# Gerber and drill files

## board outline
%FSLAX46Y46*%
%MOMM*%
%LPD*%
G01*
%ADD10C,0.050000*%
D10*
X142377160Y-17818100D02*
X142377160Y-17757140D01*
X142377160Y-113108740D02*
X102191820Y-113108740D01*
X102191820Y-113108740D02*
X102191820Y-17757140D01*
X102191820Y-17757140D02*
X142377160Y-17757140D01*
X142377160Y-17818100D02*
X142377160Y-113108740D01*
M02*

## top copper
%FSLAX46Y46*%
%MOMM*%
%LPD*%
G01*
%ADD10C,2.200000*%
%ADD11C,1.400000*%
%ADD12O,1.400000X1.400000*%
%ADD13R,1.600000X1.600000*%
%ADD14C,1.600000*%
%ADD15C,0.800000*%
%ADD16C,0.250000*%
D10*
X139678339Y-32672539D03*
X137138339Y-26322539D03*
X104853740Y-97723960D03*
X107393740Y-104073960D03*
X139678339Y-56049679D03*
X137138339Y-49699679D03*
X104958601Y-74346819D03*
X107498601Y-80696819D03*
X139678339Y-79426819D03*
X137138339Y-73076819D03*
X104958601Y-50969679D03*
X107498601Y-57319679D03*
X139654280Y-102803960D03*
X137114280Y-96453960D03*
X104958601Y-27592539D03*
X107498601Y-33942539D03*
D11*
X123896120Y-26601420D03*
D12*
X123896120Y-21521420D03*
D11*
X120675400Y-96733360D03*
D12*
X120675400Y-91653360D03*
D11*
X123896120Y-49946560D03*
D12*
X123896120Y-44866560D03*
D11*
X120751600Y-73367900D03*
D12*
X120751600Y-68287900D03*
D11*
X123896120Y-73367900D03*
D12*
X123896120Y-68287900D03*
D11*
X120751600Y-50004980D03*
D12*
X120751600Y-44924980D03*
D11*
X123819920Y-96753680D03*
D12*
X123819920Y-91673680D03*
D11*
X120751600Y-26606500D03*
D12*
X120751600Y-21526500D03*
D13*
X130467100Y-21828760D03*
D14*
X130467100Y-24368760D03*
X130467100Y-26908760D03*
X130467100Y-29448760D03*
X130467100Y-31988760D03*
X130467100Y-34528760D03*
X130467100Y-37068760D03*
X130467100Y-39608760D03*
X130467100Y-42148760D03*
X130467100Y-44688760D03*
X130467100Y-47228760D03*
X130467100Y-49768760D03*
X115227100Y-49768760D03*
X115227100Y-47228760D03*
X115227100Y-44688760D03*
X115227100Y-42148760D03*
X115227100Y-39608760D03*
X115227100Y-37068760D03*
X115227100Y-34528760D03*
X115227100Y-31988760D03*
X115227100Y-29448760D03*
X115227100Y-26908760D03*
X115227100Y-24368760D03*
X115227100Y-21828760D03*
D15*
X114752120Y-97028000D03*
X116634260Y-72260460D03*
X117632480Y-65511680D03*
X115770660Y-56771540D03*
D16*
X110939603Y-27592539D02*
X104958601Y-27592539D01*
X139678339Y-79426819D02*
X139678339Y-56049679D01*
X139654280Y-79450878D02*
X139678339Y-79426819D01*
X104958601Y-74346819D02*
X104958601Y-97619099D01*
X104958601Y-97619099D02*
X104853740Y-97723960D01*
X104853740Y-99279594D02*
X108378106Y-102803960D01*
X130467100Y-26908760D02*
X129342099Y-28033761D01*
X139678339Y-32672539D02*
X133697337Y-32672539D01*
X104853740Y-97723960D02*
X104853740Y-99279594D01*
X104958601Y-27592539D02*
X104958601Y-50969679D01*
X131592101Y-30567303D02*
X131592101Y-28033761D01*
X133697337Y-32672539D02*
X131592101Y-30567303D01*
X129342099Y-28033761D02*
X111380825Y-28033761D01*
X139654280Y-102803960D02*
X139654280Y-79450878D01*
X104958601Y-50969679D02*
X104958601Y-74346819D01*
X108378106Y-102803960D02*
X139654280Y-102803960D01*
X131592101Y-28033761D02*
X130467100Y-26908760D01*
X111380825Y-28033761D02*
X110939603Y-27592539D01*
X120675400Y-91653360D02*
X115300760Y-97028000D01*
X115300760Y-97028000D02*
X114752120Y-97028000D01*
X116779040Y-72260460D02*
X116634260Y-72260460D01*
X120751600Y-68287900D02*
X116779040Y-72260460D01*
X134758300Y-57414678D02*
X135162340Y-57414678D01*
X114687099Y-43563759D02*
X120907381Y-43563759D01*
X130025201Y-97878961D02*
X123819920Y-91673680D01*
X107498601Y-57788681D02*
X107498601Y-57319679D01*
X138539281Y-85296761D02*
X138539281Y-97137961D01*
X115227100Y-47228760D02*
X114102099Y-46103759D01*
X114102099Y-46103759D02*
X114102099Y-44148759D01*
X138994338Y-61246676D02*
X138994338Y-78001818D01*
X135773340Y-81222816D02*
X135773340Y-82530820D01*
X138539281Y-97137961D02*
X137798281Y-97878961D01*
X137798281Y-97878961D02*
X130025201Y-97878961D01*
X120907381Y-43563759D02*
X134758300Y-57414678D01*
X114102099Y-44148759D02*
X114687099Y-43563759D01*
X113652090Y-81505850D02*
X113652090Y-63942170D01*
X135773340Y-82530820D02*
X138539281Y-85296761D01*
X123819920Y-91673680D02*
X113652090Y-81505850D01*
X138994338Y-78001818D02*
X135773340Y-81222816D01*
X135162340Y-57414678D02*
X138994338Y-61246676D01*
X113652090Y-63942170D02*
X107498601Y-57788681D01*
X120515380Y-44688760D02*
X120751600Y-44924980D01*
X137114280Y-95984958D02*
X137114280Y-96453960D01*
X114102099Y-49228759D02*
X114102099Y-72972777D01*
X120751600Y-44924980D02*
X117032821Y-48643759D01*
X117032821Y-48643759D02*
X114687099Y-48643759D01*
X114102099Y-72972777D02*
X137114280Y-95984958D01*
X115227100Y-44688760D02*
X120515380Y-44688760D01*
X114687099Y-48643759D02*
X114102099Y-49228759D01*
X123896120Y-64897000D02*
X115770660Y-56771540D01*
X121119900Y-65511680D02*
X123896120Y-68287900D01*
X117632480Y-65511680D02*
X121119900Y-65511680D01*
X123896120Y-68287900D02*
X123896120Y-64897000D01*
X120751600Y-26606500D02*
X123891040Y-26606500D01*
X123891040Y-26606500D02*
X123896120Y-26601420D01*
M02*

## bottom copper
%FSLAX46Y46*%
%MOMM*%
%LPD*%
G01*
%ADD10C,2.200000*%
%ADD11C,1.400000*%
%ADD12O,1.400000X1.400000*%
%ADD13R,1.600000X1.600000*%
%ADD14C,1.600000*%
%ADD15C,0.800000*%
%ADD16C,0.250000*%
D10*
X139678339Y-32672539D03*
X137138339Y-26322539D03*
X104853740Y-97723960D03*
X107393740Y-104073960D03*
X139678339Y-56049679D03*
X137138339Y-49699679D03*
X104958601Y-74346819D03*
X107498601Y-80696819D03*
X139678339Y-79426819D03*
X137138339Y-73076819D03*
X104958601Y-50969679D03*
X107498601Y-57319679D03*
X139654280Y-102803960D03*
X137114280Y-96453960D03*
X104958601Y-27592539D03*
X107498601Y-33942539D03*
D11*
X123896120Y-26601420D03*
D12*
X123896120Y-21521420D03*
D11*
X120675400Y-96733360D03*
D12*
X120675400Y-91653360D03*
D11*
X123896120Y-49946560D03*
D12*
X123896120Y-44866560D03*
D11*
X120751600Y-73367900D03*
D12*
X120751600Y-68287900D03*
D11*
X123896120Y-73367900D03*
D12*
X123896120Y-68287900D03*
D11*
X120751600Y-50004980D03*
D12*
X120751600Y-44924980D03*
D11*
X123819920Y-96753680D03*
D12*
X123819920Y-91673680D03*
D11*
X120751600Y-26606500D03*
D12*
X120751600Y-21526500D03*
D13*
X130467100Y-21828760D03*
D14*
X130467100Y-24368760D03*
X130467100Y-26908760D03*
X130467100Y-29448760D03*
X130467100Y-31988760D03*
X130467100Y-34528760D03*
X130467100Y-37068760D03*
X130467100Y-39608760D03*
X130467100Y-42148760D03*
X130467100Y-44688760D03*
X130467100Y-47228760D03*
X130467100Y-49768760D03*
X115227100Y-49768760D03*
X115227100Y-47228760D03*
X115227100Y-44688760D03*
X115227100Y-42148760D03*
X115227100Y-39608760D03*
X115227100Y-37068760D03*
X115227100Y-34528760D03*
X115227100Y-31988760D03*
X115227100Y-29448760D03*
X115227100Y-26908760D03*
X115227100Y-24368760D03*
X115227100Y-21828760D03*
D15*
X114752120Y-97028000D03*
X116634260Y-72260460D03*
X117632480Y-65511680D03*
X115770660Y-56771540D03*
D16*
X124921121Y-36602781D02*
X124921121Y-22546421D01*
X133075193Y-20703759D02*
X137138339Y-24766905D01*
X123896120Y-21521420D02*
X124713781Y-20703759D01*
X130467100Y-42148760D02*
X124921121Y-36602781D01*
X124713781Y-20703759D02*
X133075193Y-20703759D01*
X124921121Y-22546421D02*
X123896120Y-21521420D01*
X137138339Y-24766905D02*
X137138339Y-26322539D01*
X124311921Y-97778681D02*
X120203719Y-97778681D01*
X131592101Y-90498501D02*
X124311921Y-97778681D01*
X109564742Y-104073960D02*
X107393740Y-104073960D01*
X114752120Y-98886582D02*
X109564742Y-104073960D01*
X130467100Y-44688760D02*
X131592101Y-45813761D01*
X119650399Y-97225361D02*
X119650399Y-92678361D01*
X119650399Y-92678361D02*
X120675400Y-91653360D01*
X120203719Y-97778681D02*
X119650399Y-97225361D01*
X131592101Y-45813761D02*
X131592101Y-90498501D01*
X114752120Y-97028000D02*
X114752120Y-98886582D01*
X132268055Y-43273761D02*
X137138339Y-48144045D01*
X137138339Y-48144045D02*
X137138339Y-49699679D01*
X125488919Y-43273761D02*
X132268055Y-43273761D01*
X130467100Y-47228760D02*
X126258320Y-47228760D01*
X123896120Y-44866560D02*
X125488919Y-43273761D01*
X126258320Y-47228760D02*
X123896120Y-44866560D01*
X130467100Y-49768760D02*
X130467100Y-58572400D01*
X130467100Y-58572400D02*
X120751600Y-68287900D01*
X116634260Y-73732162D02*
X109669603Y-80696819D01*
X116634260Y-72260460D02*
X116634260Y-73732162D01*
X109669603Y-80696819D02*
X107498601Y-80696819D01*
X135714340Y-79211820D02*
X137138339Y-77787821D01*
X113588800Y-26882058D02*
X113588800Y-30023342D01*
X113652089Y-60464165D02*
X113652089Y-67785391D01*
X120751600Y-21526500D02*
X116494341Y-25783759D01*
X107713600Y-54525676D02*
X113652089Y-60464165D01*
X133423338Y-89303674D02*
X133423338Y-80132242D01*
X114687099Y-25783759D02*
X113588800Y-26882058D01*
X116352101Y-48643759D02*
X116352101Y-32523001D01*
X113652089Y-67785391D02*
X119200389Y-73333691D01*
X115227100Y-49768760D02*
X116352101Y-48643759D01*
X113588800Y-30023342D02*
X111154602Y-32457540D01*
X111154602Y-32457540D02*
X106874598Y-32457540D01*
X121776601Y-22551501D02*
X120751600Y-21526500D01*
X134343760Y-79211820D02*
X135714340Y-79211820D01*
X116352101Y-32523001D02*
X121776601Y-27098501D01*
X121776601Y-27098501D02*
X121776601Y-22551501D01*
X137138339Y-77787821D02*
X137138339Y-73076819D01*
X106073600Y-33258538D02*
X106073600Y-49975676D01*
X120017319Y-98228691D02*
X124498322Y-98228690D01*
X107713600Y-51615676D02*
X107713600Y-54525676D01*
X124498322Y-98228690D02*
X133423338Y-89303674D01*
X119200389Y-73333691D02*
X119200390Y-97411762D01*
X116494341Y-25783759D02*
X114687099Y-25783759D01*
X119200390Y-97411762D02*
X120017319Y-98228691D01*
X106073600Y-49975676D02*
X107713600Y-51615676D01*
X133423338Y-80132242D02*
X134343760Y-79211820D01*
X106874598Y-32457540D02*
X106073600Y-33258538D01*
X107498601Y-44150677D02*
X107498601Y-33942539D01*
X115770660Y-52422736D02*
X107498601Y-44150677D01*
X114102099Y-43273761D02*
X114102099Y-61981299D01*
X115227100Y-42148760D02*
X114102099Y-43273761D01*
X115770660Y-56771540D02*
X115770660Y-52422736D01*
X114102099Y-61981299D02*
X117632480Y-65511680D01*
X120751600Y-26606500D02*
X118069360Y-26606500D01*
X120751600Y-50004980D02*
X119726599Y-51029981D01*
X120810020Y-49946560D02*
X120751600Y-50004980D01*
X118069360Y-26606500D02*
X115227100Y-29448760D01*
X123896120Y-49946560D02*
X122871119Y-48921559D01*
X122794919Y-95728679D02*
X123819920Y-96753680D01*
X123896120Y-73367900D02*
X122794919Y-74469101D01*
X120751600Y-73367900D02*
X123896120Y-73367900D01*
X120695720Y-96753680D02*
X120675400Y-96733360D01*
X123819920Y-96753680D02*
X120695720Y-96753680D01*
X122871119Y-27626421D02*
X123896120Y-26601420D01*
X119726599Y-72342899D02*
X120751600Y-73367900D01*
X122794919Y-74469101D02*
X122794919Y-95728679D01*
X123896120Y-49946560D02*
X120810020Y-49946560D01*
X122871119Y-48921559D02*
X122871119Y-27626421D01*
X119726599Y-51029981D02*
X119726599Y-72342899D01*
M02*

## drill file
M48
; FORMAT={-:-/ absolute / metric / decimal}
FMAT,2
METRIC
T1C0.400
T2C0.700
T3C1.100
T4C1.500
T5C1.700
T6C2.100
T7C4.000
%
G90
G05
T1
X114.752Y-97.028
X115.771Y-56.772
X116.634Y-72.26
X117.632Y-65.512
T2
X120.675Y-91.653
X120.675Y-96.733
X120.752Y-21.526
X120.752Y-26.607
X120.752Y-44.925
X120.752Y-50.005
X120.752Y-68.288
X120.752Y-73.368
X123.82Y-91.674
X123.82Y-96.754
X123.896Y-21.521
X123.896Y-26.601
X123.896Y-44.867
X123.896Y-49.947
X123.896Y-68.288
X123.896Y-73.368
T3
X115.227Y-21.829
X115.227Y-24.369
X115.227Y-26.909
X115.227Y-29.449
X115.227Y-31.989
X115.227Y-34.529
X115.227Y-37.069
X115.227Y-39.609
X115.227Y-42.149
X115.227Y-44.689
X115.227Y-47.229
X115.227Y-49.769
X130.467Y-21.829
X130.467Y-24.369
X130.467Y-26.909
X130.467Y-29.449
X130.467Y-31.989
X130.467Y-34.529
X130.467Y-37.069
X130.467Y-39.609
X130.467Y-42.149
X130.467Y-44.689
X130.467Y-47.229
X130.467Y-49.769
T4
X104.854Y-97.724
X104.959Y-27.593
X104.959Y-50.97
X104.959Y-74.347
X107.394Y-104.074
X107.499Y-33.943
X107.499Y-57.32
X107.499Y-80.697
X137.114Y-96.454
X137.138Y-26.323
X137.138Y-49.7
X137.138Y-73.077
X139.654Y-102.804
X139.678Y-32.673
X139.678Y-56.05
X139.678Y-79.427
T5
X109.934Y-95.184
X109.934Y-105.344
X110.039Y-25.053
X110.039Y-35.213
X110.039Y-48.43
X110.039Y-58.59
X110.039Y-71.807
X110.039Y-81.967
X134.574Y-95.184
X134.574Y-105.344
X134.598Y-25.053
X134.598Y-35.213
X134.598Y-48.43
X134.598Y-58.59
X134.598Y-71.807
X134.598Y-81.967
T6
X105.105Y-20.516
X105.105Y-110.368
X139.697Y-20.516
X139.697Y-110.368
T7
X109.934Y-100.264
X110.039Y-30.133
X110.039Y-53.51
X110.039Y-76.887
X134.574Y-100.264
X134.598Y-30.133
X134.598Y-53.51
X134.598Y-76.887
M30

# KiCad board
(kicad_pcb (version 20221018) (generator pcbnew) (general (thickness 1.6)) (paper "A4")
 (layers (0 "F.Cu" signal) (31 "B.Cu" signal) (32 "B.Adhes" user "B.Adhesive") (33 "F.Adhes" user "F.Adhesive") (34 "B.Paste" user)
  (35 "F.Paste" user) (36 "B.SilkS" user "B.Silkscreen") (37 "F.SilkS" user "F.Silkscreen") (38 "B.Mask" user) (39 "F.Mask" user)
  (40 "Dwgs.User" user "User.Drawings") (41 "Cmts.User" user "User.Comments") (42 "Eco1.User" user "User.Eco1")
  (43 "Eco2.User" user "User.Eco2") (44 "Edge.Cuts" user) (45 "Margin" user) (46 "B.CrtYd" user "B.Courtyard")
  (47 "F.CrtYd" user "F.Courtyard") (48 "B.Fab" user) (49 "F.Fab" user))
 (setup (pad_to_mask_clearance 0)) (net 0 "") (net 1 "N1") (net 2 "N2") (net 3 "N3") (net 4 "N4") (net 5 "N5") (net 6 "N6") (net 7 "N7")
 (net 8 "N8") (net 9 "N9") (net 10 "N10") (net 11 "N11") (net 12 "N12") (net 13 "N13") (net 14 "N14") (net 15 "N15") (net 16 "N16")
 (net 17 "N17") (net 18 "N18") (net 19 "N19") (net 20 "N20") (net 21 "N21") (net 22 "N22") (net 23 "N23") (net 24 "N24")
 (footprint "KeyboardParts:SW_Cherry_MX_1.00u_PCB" (layer "F.Cu") (at 139.678339 32.672539 -90)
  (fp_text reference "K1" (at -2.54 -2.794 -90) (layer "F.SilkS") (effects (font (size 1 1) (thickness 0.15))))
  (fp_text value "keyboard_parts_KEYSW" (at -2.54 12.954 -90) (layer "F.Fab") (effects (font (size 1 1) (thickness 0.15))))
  (pad "" np_thru_hole circle (at -7.62 5.08 270) (size 1.7 1.7) (drill 1.7) (layers "*.Cu" "*.Mask"))
  (pad "" np_thru_hole circle (at -2.54 5.08 270) (size 4 4) (drill 4) (layers "*.Cu" "*.Mask"))
  (pad "" np_thru_hole circle (at 2.54 5.08 270) (size 1.7 1.7) (drill 1.7) (layers "*.Cu" "*.Mask"))
  (pad "1" thru_hole circle (at 0 0 270) (size 2.2 2.2) (drill 1.5) (layers "*.Cu" "*.Mask") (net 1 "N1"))
  (pad "2" thru_hole circle (at -6.35 2.54 270) (size 2.2 2.2) (drill 1.5) (layers "*.Cu" "*.Mask") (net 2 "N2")))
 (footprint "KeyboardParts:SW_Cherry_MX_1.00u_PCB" (layer "F.Cu") (at 104.85374 97.72396 90)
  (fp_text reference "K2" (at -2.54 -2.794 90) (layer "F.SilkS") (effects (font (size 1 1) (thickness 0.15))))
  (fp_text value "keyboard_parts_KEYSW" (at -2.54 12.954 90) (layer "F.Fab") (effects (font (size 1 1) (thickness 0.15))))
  (pad "" np_thru_hole circle (at -7.62 5.08 90) (size 1.7 1.7) (drill 1.7) (layers "*.Cu" "*.Mask"))
  (pad "" np_thru_hole circle (at -2.54 5.08 90) (size 4 4) (drill 4) (layers "*.Cu" "*.Mask"))
  (pad "" np_thru_hole circle (at 2.54 5.08 90) (size 1.7 1.7) (drill 1.7) (layers "*.Cu" "*.Mask"))
  (pad "1" thru_hole circle (at 0 0 90) (size 2.2 2.2) (drill 1.5) (layers "*.Cu" "*.Mask") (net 1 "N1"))
  (pad "2" thru_hole circle (at -6.35 2.54 90) (size 2.2 2.2) (drill 1.5) (layers "*.Cu" "*.Mask") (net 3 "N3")))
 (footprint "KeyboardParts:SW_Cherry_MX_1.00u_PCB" (layer "F.Cu") (at 139.678339 56.049679 -90)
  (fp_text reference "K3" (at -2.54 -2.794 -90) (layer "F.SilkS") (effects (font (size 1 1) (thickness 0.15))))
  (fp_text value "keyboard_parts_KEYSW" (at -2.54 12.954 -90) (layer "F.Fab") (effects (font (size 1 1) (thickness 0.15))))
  (pad "" np_thru_hole circle (at -7.62 5.08 270) (size 1.7 1.7) (drill 1.7) (layers "*.Cu" "*.Mask"))
  (pad "" np_thru_hole circle (at -2.54 5.08 270) (size 4 4) (drill 4) (layers "*.Cu" "*.Mask"))
  (pad "" np_thru_hole circle (at 2.54 5.08 270) (size 1.7 1.7) (drill 1.7) (layers "*.Cu" "*.Mask"))
  (pad "1" thru_hole circle (at 0 0 270) (size 2.2 2.2) (drill 1.5) (layers "*.Cu" "*.Mask") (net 1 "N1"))
  (pad "2" thru_hole circle (at -6.35 2.54 270) (size 2.2 2.2) (drill 1.5) (layers "*.Cu" "*.Mask") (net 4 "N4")))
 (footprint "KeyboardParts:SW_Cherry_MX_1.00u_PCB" (layer "F.Cu") (at 104.958601 74.346819 90)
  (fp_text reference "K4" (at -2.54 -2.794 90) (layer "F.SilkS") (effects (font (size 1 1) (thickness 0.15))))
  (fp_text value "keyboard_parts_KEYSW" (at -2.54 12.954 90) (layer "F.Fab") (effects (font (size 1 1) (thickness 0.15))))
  (pad "" np_thru_hole circle (at -7.62 5.08 90) (size 1.7 1.7) (drill 1.7) (layers "*.Cu" "*.Mask"))
  (pad "" np_thru_hole circle (at -2.54 5.08 90) (size 4 4) (drill 4) (layers "*.Cu" "*.Mask"))
  (pad "" np_thru_hole circle (at 2.54 5.08 90) (size 1.7 1.7) (drill 1.7) (layers "*.Cu" "*.Mask"))
  (pad "1" thru_hole circle (at 0 0 90) (size 2.2 2.2) (drill 1.5) (layers "*.Cu" "*.Mask") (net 1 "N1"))
  (pad "2" thru_hole circle (at -6.35 2.54 90) (size 2.2 2.2) (drill 1.5) (layers "*.Cu" "*.Mask") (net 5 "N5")))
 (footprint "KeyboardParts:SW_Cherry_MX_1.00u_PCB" (layer "F.Cu") (at 139.678339 79.426819 -90)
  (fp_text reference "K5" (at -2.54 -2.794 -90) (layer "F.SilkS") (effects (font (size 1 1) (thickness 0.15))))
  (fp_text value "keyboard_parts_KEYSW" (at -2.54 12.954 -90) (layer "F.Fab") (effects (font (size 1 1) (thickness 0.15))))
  (pad "" np_thru_hole circle (at -7.62 5.08 270) (size 1.7 1.7) (drill 1.7) (layers "*.Cu" "*.Mask"))
  (pad "" np_thru_hole circle (at -2.54 5.08 270) (size 4 4) (drill 4) (layers "*.Cu" "*.Mask"))
  (pad "" np_thru_hole circle (at 2.54 5.08 270) (size 1.7 1.7) (drill 1.7) (layers "*.Cu" "*.Mask"))
  (pad "1" thru_hole circle (at 0 0 270) (size 2.2 2.2) (drill 1.5) (layers "*.Cu" "*.Mask") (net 1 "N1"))
  (pad "2" thru_hole circle (at -6.35 2.54 270) (size 2.2 2.2) (drill 1.5) (layers "*.Cu" "*.Mask") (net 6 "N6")))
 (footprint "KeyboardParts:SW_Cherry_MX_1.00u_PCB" (layer "F.Cu") (at 104.958601 50.969679 90)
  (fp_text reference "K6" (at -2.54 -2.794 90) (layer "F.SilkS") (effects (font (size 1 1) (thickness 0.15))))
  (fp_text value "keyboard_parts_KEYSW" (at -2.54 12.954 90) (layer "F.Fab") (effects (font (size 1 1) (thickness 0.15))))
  (pad "" np_thru_hole circle (at -7.62 5.08 90) (size 1.7 1.7) (drill 1.7) (layers "*.Cu" "*.Mask"))
  (pad "" np_thru_hole circle (at -2.54 5.08 90) (size 4 4) (drill 4) (layers "*.Cu" "*.Mask"))
  (pad "" np_thru_hole circle (at 2.54 5.08 90) (size 1.7 1.7) (drill 1.7) (layers "*.Cu" "*.Mask"))
  (pad "1" thru_hole circle (at 0 0 90) (size 2.2 2.2) (drill 1.5) (layers "*.Cu" "*.Mask") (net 1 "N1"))
  (pad "2" thru_hole circle (at -6.35 2.54 90) (size 2.2 2.2) (drill 1.5) (layers "*.Cu" "*.Mask") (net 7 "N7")))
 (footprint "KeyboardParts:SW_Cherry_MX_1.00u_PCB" (layer "F.Cu") (at 139.65428 102.80396 -90)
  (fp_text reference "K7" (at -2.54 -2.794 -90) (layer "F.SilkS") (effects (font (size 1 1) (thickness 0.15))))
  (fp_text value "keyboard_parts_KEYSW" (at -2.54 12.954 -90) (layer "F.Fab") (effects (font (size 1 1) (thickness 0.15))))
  (pad "" np_thru_hole circle (at -7.62 5.08 270) (size 1.7 1.7) (drill 1.7) (layers "*.Cu" "*.Mask"))
  (pad "" np_thru_hole circle (at -2.54 5.08 270) (size 4 4) (drill 4) (layers "*.Cu" "*.Mask"))
  (pad "" np_thru_hole circle (at 2.54 5.08 270) (size 1.7 1.7) (drill 1.7) (layers "*.Cu" "*.Mask"))
  (pad "1" thru_hole circle (at 0 0 270) (size 2.2 2.2) (drill 1.5) (layers "*.Cu" "*.Mask") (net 1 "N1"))
  (pad "2" thru_hole circle (at -6.35 2.54 270) (size 2.2 2.2) (drill 1.5) (layers "*.Cu" "*.Mask") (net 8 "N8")))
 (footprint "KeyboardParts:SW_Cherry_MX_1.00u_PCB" (layer "F.Cu") (at 104.958601 27.592539 90)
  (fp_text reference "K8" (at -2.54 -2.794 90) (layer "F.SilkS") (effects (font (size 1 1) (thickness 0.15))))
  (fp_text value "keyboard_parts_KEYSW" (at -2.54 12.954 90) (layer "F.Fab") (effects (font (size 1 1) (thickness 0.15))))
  (pad "" np_thru_hole circle (at -7.62 5.08 90) (size 1.7 1.7) (drill 1.7) (layers "*.Cu" "*.Mask"))
  (pad "" np_thru_hole circle (at -2.54 5.08 90) (size 4 4) (drill 4) (layers "*.Cu" "*.Mask"))
  (pad "" np_thru_hole circle (at 2.54 5.08 90) (size 1.7 1.7) (drill 1.7) (layers "*.Cu" "*.Mask"))
  (pad "1" thru_hole circle (at 0 0 90) (size 2.2 2.2) (drill 1.5) (layers "*.Cu" "*.Mask") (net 1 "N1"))
  (pad "2" thru_hole circle (at -6.35 2.54 90) (size 2.2 2.2) (drill 1.5) (layers "*.Cu" "*.Mask") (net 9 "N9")))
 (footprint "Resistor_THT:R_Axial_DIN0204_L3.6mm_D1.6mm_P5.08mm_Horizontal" (layer "F.Cu") (at 123.89612 26.60142 90)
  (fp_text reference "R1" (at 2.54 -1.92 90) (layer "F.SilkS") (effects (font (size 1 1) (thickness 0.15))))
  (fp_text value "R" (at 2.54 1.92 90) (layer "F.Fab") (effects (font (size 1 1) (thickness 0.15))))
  (pad "1" thru_hole circle (at 0 0 90) (size 1.4 1.4) (drill 0.7) (layers "*.Cu" "*.Mask") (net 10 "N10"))
  (pad "2" thru_hole oval (at 5.08 0 90) (size 1.4 1.4) (drill 0.7) (layers "*.Cu" "*.Mask") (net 2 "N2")))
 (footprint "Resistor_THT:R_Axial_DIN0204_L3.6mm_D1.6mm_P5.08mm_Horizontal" (layer "F.Cu") (at 120.6754 96.73336 90)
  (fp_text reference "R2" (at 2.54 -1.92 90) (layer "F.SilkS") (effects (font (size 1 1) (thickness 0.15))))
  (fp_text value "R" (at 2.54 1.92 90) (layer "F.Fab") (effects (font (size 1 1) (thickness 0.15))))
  (pad "1" thru_hole circle (at 0 0 90) (size 1.4 1.4) (drill 0.7) (layers "*.Cu" "*.Mask") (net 10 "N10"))
  (pad "2" thru_hole oval (at 5.08 0 90) (size 1.4 1.4) (drill 0.7) (layers "*.Cu" "*.Mask") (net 3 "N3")))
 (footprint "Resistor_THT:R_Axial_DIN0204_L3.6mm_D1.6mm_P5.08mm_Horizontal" (layer "F.Cu") (at 123.89612 49.94656 90)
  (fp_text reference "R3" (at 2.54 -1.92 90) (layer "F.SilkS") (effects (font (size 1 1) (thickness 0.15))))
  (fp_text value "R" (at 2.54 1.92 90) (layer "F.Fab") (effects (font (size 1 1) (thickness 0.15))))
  (pad "1" thru_hole circle (at 0 0 90) (size 1.4 1.4) (drill 0.7) (layers "*.Cu" "*.Mask") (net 10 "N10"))
  (pad "2" thru_hole oval (at 5.08 0 90) (size 1.4 1.4) (drill 0.7) (layers "*.Cu" "*.Mask") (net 4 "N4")))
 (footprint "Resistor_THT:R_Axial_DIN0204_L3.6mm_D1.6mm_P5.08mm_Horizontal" (layer "F.Cu") (at 120.7516 73.3679 90)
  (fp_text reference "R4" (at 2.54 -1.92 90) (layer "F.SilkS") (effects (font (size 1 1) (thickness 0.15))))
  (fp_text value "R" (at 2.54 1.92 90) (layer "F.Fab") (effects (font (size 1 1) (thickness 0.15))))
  (pad "1" thru_hole circle (at 0 0 90) (size 1.4 1.4) (drill 0.7) (layers "*.Cu" "*.Mask") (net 10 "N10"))
  (pad "2" thru_hole oval (at 5.08 0 90) (size 1.4 1.4) (drill 0.7) (layers "*.Cu" "*.Mask") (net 5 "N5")))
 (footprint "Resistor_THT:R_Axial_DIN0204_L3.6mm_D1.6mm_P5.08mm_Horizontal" (layer "F.Cu") (at 123.89612 73.3679 90)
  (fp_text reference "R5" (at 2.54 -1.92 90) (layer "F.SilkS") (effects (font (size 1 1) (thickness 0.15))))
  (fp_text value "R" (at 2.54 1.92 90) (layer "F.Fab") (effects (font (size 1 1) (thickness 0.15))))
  (pad "1" thru_hole circle (at 0 0 90) (size 1.4 1.4) (drill 0.7) (layers "*.Cu" "*.Mask") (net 10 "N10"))
  (pad "2" thru_hole oval (at 5.08 0 90) (size 1.4 1.4) (drill 0.7) (layers "*.Cu" "*.Mask") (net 9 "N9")))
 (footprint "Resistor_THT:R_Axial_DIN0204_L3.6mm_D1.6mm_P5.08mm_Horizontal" (layer "F.Cu") (at 120.7516 50.00498 90)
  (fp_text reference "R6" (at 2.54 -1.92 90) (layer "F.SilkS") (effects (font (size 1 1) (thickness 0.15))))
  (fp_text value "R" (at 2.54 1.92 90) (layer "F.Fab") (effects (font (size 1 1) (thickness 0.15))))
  (pad "1" thru_hole circle (at 0 0 90) (size 1.4 1.4) (drill 0.7) (layers "*.Cu" "*.Mask") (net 10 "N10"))
  (pad "2" thru_hole oval (at 5.08 0 90) (size 1.4 1.4) (drill 0.7) (layers "*.Cu" "*.Mask") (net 8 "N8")))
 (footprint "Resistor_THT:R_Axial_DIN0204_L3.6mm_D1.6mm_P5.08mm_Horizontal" (layer "F.Cu") (at 123.81992 96.75368 90)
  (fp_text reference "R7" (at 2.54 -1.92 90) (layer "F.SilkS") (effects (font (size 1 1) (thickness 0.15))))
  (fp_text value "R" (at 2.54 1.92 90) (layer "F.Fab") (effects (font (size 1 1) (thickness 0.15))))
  (pad "1" thru_hole circle (at 0 0 90) (size 1.4 1.4) (drill 0.7) (layers "*.Cu" "*.Mask") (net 10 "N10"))
  (pad "2" thru_hole oval (at 5.08 0 90) (size 1.4 1.4) (drill 0.7) (layers "*.Cu" "*.Mask") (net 7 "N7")))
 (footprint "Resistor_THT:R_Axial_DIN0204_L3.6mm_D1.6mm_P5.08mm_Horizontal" (layer "F.Cu") (at 120.7516 26.6065 90)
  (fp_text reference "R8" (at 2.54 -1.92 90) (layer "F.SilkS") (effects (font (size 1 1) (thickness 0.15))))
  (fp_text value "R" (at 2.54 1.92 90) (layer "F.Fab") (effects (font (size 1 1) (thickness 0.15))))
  (pad "1" thru_hole circle (at 0 0 90) (size 1.4 1.4) (drill 0.7) (layers "*.Cu" "*.Mask") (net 10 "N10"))
  (pad "2" thru_hole oval (at 5.08 0 90) (size 1.4 1.4) (drill 0.7) (layers "*.Cu" "*.Mask") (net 6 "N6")))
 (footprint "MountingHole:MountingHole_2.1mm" (layer "F.Cu") (at 139.69746 110.36808)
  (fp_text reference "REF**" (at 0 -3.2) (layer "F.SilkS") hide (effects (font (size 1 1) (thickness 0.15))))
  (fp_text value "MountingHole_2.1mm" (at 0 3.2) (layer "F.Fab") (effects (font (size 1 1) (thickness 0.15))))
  (pad "" np_thru_hole circle (at 0 0) (size 2.1 2.1) (drill 2.1) (layers "*.Cu" "*.Mask")))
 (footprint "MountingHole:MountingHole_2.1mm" (layer "F.Cu") (at 105.1052 110.36808)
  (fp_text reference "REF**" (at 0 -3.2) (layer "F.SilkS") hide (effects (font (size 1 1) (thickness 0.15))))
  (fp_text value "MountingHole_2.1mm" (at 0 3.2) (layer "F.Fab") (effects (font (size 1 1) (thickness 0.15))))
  (pad "" np_thru_hole circle (at 0 0) (size 2.1 2.1) (drill 2.1) (layers "*.Cu" "*.Mask")))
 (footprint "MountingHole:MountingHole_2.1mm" (layer "F.Cu") (at 105.1052 20.51558)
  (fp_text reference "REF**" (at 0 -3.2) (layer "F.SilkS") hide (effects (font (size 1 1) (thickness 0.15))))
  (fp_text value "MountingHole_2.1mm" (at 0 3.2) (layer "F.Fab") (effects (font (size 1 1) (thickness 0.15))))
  (pad "" np_thru_hole circle (at 0 0) (size 2.1 2.1) (drill 2.1) (layers "*.Cu" "*.Mask")))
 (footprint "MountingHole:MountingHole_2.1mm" (layer "F.Cu") (at 139.69746 20.51558)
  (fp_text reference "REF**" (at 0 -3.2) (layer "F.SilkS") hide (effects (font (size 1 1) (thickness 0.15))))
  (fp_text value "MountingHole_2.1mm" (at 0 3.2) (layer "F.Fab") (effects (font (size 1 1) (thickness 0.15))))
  (pad "" np_thru_hole circle (at 0 0) (size 2.1 2.1) (drill 2.1) (layers "*.Cu" "*.Mask")))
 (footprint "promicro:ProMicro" (layer "B.Cu") (at 122.8471 35.79876 -90)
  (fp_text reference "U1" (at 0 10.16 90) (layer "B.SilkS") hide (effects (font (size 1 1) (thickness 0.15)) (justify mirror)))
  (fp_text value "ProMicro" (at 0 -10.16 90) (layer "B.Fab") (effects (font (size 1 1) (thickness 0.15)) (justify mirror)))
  (pad "1" thru_hole rect (at -13.97 -7.62 270) (size 1.6 1.6) (drill 1.1) (layers "*.Cu" "*.Mask" "B.SilkS") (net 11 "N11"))
  (pad "2" thru_hole circle (at -11.43 -7.62 270) (size 1.6 1.6) (drill 1.1) (layers "*.Cu" "*.Mask" "B.SilkS") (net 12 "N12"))
  (pad "3" thru_hole circle (at -8.89 -7.62 270) (size 1.6 1.6) (drill 1.1) (layers "*.Cu" "*.Mask" "B.SilkS") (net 1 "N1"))
  (pad "4" thru_hole circle (at -6.35 -7.62 270) (size 1.6 1.6) (drill 1.1) (layers "*.Cu" "*.Mask" "B.SilkS") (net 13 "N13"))
  (pad "5" thru_hole circle (at -3.81 -7.62 270) (size 1.6 1.6) (drill 1.1) (layers "*.Cu" "*.Mask" "B.SilkS") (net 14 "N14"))
  (pad "6" thru_hole circle (at -1.27 -7.62 270) (size 1.6 1.6) (drill 1.1) (layers "*.Cu" "*.Mask" "B.SilkS") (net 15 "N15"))
  (pad "7" thru_hole circle (at 1.27 -7.62 270) (size 1.6 1.6) (drill 1.1) (layers "*.Cu" "*.Mask" "B.SilkS") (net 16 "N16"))
  (pad "8" thru_hole circle (at 3.81 -7.62 270) (size 1.6 1.6) (drill 1.1) (layers "*.Cu" "*.Mask" "B.SilkS") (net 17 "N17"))
  (pad "9" thru_hole circle (at 6.35 -7.62 270) (size 1.6 1.6) (drill 1.1) (layers "*.Cu" "*.Mask" "B.SilkS") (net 2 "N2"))
  (pad "10" thru_hole circle (at 8.89 -7.62 270) (size 1.6 1.6) (drill 1.1) (layers "*.Cu" "*.Mask" "B.SilkS") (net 3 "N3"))
  (pad "11" thru_hole circle (at 11.43 -7.62 270) (size 1.6 1.6) (drill 1.1) (layers "*.Cu" "*.Mask" "B.SilkS") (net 4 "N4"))
  (pad "12" thru_hole circle (at 13.97 -7.62 270) (size 1.6 1.6) (drill 1.1) (layers "*.Cu" "*.Mask" "B.SilkS") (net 5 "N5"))
  (pad "13" thru_hole circle (at 13.97 7.62 270) (size 1.6 1.6) (drill 1.1) (layers "*.Cu" "*.Mask" "B.SilkS") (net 6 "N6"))
  (pad "14" thru_hole circle (at 11.43 7.62 270) (size 1.6 1.6) (drill 1.1) (layers "*.Cu" "*.Mask" "B.SilkS") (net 7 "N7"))
  (pad "15" thru_hole circle (at 8.89 7.62 270) (size 1.6 1.6) (drill 1.1) (layers "*.Cu" "*.Mask" "B.SilkS") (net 8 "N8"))
  (pad "16" thru_hole circle (at 6.35 7.62 270) (size 1.6 1.6) (drill 1.1) (layers "*.Cu" "*.Mask" "B.SilkS") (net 9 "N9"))
  (pad "17" thru_hole circle (at 3.81 7.62 270) (size 1.6 1.6) (drill 1.1) (layers "*.Cu" "*.Mask" "B.SilkS") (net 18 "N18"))
  (pad "18" thru_hole circle (at 1.27 7.62 270) (size 1.6 1.6) (drill 1.1) (layers "*.Cu" "*.Mask" "B.SilkS") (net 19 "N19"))
  (pad "19" thru_hole circle (at -1.27 7.62 270) (size 1.6 1.6) (drill 1.1) (layers "*.Cu" "*.Mask" "B.SilkS") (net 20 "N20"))
  (pad "20" thru_hole circle (at -3.81 7.62 270) (size 1.6 1.6) (drill 1.1) (layers "*.Cu" "*.Mask" "B.SilkS") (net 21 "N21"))
  (pad "21" thru_hole circle (at -6.35 7.62 270) (size 1.6 1.6) (drill 1.1) (layers "*.Cu" "*.Mask" "B.SilkS") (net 10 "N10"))
  (pad "22" thru_hole circle (at -8.89 7.62 270) (size 1.6 1.6) (drill 1.1) (layers "*.Cu" "*.Mask" "B.SilkS") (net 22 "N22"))
  (pad "23" thru_hole circle (at -11.43 7.62 270) (size 1.6 1.6) (drill 1.1) (layers "*.Cu" "*.Mask" "B.SilkS") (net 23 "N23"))
  (pad "24" thru_hole circle (at -13.97 7.62 270) (size 1.6 1.6) (drill 1.1) (layers "*.Cu" "*.Mask" "B.SilkS") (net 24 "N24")))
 (gr_line (start 142.37716 17.8181) (end 142.37716 17.75714) (stroke (width 0.05) (type solid)) (layer "Edge.Cuts"))
 (gr_line (start 142.37716 113.10874) (end 102.19182 113.10874) (stroke (width 0.05) (type solid)) (layer "Edge.Cuts"))
 (gr_line (start 102.19182 113.10874) (end 102.19182 17.75714) (stroke (width 0.05) (type solid)) (layer "Edge.Cuts"))
 (gr_line (start 102.19182 17.75714) (end 142.37716 17.75714) (stroke (width 0.05) (type solid)) (layer "Edge.Cuts"))
 (gr_line (start 142.37716 17.8181) (end 142.37716 113.10874) (stroke (width 0.05) (type solid)) (layer "Edge.Cuts"))
 (segment (start 110.939603 27.592539) (end 104.958601 27.592539) (width 0.25) (layer "F.Cu") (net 1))
 (segment (start 139.678339 79.426819) (end 139.678339 56.049679) (width 0.25) (layer "F.Cu") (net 1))
 (segment (start 139.65428 79.450878) (end 139.678339 79.426819) (width 0.25) (layer "F.Cu") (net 1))
 (segment (start 104.958601 74.346819) (end 104.958601 97.619099) (width 0.25) (layer "F.Cu") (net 1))
 (segment (start 104.958601 97.619099) (end 104.85374 97.72396) (width 0.25) (layer "F.Cu") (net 1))
 (segment (start 104.85374 99.279594) (end 108.378106 102.80396) (width 0.25) (layer "F.Cu") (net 1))
 (segment (start 130.4671 26.90876) (end 129.342099 28.033761) (width 0.25) (layer "F.Cu") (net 1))
 (segment (start 139.678339 32.672539) (end 133.697337 32.672539) (width 0.25) (layer "F.Cu") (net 1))
 (segment (start 104.85374 97.72396) (end 104.85374 99.279594) (width 0.25) (layer "F.Cu") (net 1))
 (segment (start 104.958601 27.592539) (end 104.958601 50.969679) (width 0.25) (layer "F.Cu") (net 1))
 (segment (start 131.592101 30.567303) (end 131.592101 28.033761) (width 0.25) (layer "F.Cu") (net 1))
 (segment (start 133.697337 32.672539) (end 131.592101 30.567303) (width 0.25) (layer "F.Cu") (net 1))
 (segment (start 129.342099 28.033761) (end 111.380825 28.033761) (width 0.25) (layer "F.Cu") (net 1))
 (segment (start 139.65428 102.80396) (end 139.65428 79.450878) (width 0.25) (layer "F.Cu") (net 1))
 (segment (start 104.958601 50.969679) (end 104.958601 74.346819) (width 0.25) (layer "F.Cu") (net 1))
 (segment (start 108.378106 102.80396) (end 139.65428 102.80396) (width 0.25) (layer "F.Cu") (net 1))
 (segment (start 131.592101 28.033761) (end 130.4671 26.90876) (width 0.25) (layer "F.Cu") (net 1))
 (segment (start 111.380825 28.033761) (end 110.939603 27.592539) (width 0.25) (layer "F.Cu") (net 1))
 (segment (start 124.921121 36.602781) (end 124.921121 22.546421) (width 0.25) (layer "B.Cu") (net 2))
 (segment (start 133.075193 20.703759) (end 137.138339 24.766905) (width 0.25) (layer "B.Cu") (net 2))
 (segment (start 123.89612 21.52142) (end 124.713781 20.703759) (width 0.25) (layer "B.Cu") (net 2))
 (segment (start 130.4671 42.14876) (end 124.921121 36.602781) (width 0.25) (layer "B.Cu") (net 2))
 (segment (start 124.713781 20.703759) (end 133.075193 20.703759) (width 0.25) (layer "B.Cu") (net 2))
 (segment (start 124.921121 22.546421) (end 123.89612 21.52142) (width 0.25) (layer "B.Cu") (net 2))
 (segment (start 137.138339 24.766905) (end 137.138339 26.322539) (width 0.25) (layer "B.Cu") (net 2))
 (segment (start 120.6754 91.65336) (end 115.30076 97.028) (width 0.25) (layer "F.Cu") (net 3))
 (segment (start 115.30076 97.028) (end 114.75212 97.028) (width 0.25) (layer "F.Cu") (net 3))
 (via (at 114.75212 97.028) (size 0.8) (drill 0.4) (layers "F.Cu" "B.Cu") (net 3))
 (segment (start 124.311921 97.778681) (end 120.203719 97.778681) (width 0.25) (layer "B.Cu") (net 3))
 (segment (start 131.592101 90.498501) (end 124.311921 97.778681) (width 0.25) (layer "B.Cu") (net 3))
 (segment (start 109.564742 104.07396) (end 107.39374 104.07396) (width 0.25) (layer "B.Cu") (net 3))
 (segment (start 114.75212 98.886582) (end 109.564742 104.07396) (width 0.25) (layer "B.Cu") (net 3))
 (segment (start 130.4671 44.68876) (end 131.592101 45.813761) (width 0.25) (layer "B.Cu") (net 3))
 (segment (start 119.650399 97.225361) (end 119.650399 92.678361) (width 0.25) (layer "B.Cu") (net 3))
 (segment (start 119.650399 92.678361) (end 120.6754 91.65336) (width 0.25) (layer "B.Cu") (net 3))
 (segment (start 120.203719 97.778681) (end 119.650399 97.225361) (width 0.25) (layer "B.Cu") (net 3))
 (segment (start 131.592101 45.813761) (end 131.592101 90.498501) (width 0.25) (layer "B.Cu") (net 3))
 (segment (start 114.75212 97.028) (end 114.75212 98.886582) (width 0.25) (layer "B.Cu") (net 3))
 (segment (start 132.268055 43.273761) (end 137.138339 48.144045) (width 0.25) (layer "B.Cu") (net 4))
 (segment (start 137.138339 48.144045) (end 137.138339 49.699679) (width 0.25) (layer "B.Cu") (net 4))
 (segment (start 125.488919 43.273761) (end 132.268055 43.273761) (width 0.25) (layer "B.Cu") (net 4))
 (segment (start 130.4671 47.22876) (end 126.25832 47.22876) (width 0.25) (layer "B.Cu") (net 4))
 (segment (start 123.89612 44.86656) (end 125.488919 43.273761) (width 0.25) (layer "B.Cu") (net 4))
 (segment (start 126.25832 47.22876) (end 123.89612 44.86656) (width 0.25) (layer "B.Cu") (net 4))
 (segment (start 116.77904 72.26046) (end 116.63426 72.26046) (width 0.25) (layer "F.Cu") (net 5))
 (segment (start 120.7516 68.2879) (end 116.77904 72.26046) (width 0.25) (layer "F.Cu") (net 5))
 (via (at 116.63426 72.26046) (size 0.8) (drill 0.4) (layers "F.Cu" "B.Cu") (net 5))
 (segment (start 130.4671 49.76876) (end 130.4671 58.5724) (width 0.25) (layer "B.Cu") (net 5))
 (segment (start 130.4671 58.5724) (end 120.7516 68.2879) (width 0.25) (layer "B.Cu") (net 5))
 (segment (start 116.63426 73.732162) (end 109.669603 80.696819) (width 0.25) (layer "B.Cu") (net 5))
 (segment (start 116.63426 72.26046) (end 116.63426 73.732162) (width 0.25) (layer "B.Cu") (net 5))
 (segment (start 109.669603 80.696819) (end 107.498601 80.696819) (width 0.25) (layer "B.Cu") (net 5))
 (segment (start 135.71434 79.21182) (end 137.138339 77.787821) (width 0.25) (layer "B.Cu") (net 6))
 (segment (start 113.5888 26.882058) (end 113.5888 30.023342) (width 0.25) (layer "B.Cu") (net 6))
 (segment (start 113.652089 60.464165) (end 113.652089 67.785391) (width 0.25) (layer "B.Cu") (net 6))
 (segment (start 120.7516 21.5265) (end 116.494341 25.783759) (width 0.25) (layer "B.Cu") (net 6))
 (segment (start 107.7136 54.525676) (end 113.652089 60.464165) (width 0.25) (layer "B.Cu") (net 6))
 (segment (start 133.423338 89.303674) (end 133.423338 80.132242) (width 0.25) (layer "B.Cu") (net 6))
 (segment (start 114.687099 25.783759) (end 113.5888 26.882058) (width 0.25) (layer "B.Cu") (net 6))
 (segment (start 116.352101 48.643759) (end 116.352101 32.523001) (width 0.25) (layer "B.Cu") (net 6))
 (segment (start 113.652089 67.785391) (end 119.200389 73.333691) (width 0.25) (layer "B.Cu") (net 6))
 (segment (start 115.2271 49.76876) (end 116.352101 48.643759) (width 0.25) (layer "B.Cu") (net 6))
 (segment (start 113.5888 30.023342) (end 111.154602 32.45754) (width 0.25) (layer "B.Cu") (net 6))
 (segment (start 111.154602 32.45754) (end 106.874598 32.45754) (width 0.25) (layer "B.Cu") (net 6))
 (segment (start 121.776601 22.551501) (end 120.7516 21.5265) (width 0.25) (layer "B.Cu") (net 6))
 (segment (start 134.34376 79.21182) (end 135.71434 79.21182) (width 0.25) (layer "B.Cu") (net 6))
 (segment (start 116.352101 32.523001) (end 121.776601 27.098501) (width 0.25) (layer "B.Cu") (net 6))
 (segment (start 121.776601 27.098501) (end 121.776601 22.551501) (width 0.25) (layer "B.Cu") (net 6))
 (segment (start 137.138339 77.787821) (end 137.138339 73.076819) (width 0.25) (layer "B.Cu") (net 6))
 (segment (start 106.0736 33.258538) (end 106.0736 49.975676) (width 0.25) (layer "B.Cu") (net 6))
 (segment (start 120.017319 98.228691) (end 124.498322 98.22869) (width 0.25) (layer "B.Cu") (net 6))
 (segment (start 107.7136 51.615676) (end 107.7136 54.525676) (width 0.25) (layer "B.Cu") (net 6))
 (segment (start 124.498322 98.22869) (end 133.423338 89.303674) (width 0.25) (layer "B.Cu") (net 6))
 (segment (start 119.200389 73.333691) (end 119.20039 97.411762) (width 0.25) (layer "B.Cu") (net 6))
 (segment (start 116.494341 25.783759) (end 114.687099 25.783759) (width 0.25) (layer "B.Cu") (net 6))
 (segment (start 119.20039 97.411762) (end 120.017319 98.228691) (width 0.25) (layer "B.Cu") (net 6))
 (segment (start 106.0736 49.975676) (end 107.7136 51.615676) (width 0.25) (layer "B.Cu") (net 6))
 (segment (start 133.423338 80.132242) (end 134.34376 79.21182) (width 0.25) (layer "B.Cu") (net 6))
 (segment (start 106.874598 32.45754) (end 106.0736 33.258538) (width 0.25) (layer "B.Cu") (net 6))
 (segment (start 134.7583 57.414678) (end 135.16234 57.414678) (width 0.25) (layer "F.Cu") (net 7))
 (segment (start 114.687099 43.563759) (end 120.907381 43.563759) (width 0.25) (layer "F.Cu") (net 7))
 (segment (start 130.025201 97.878961) (end 123.81992 91.67368) (width 0.25) (layer "F.Cu") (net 7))
 (segment (start 107.498601 57.788681) (end 107.498601 57.319679) (width 0.25) (layer "F.Cu") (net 7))
 (segment (start 138.539281 85.296761) (end 138.539281 97.137961) (width 0.25) (layer "F.Cu") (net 7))
 (segment (start 115.2271 47.22876) (end 114.102099 46.103759) (width 0.25) (layer "F.Cu") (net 7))
 (segment (start 114.102099 46.103759) (end 114.102099 44.148759) (width 0.25) (layer "F.Cu") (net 7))
 (segment (start 138.994338 61.246676) (end 138.994338 78.001818) (width 0.25) (layer "F.Cu") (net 7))
 (segment (start 135.77334 81.222816) (end 135.77334 82.53082) (width 0.25) (layer "F.Cu") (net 7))
 (segment (start 138.539281 97.137961) (end 137.798281 97.878961) (width 0.25) (layer "F.Cu") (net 7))
 (segment (start 137.798281 97.878961) (end 130.025201 97.878961) (width 0.25) (layer "F.Cu") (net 7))
 (segment (start 120.907381 43.563759) (end 134.7583 57.414678) (width 0.25) (layer "F.Cu") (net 7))
 (segment (start 114.102099 44.148759) (end 114.687099 43.563759) (width 0.25) (layer "F.Cu") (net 7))
 (segment (start 113.65209 81.50585) (end 113.65209 63.94217) (width 0.25) (layer "F.Cu") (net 7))
 (segment (start 135.77334 82.53082) (end 138.539281 85.296761) (width 0.25) (layer "F.Cu") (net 7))
 (segment (start 123.81992 91.67368) (end 113.65209 81.50585) (width 0.25) (layer "F.Cu") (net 7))
 (segment (start 138.994338 78.001818) (end 135.77334 81.222816) (width 0.25) (layer "F.Cu") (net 7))
 (segment (start 135.16234 57.414678) (end 138.994338 61.246676) (width 0.25) (layer "F.Cu") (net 7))
 (segment (start 113.65209 63.94217) (end 107.498601 57.788681) (width 0.25) (layer "F.Cu") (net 7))
 (segment (start 120.51538 44.68876) (end 120.7516 44.92498) (width 0.25) (layer "F.Cu") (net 8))
 (segment (start 137.11428 95.984958) (end 137.11428 96.45396) (width 0.25) (layer "F.Cu") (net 8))
 (segment (start 114.102099 49.228759) (end 114.102099 72.972777) (width 0.25) (layer "F.Cu") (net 8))
 (segment (start 120.7516 44.92498) (end 117.032821 48.643759) (width 0.25) (layer "F.Cu") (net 8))
 (segment (start 117.032821 48.643759) (end 114.687099 48.643759) (width 0.25) (layer "F.Cu") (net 8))
 (segment (start 114.102099 72.972777) (end 137.11428 95.984958) (width 0.25) (layer "F.Cu") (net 8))
 (segment (start 115.2271 44.68876) (end 120.51538 44.68876) (width 0.25) (layer "F.Cu") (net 8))
 (segment (start 114.687099 48.643759) (end 114.102099 49.228759) (width 0.25) (layer "F.Cu") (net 8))
 (segment (start 123.89612 64.897) (end 115.77066 56.77154) (width 0.25) (layer "F.Cu") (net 9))
 (segment (start 121.1199 65.51168) (end 123.89612 68.2879) (width 0.25) (layer "F.Cu") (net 9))
 (segment (start 117.63248 65.51168) (end 121.1199 65.51168) (width 0.25) (layer "F.Cu") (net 9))
 (segment (start 123.89612 68.2879) (end 123.89612 64.897) (width 0.25) (layer "F.Cu") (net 9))
 (via (at 117.63248 65.51168) (size 0.8) (drill 0.4) (layers "F.Cu" "B.Cu") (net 9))
 (via (at 115.77066 56.77154) (size 0.8) (drill 0.4) (layers "F.Cu" "B.Cu") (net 9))
 (segment (start 107.498601 44.150677) (end 107.498601 33.942539) (width 0.25) (layer "B.Cu") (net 9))
 (segment (start 115.77066 52.422736) (end 107.498601 44.150677) (width 0.25) (layer "B.Cu") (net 9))
 (segment (start 114.102099 43.273761) (end 114.102099 61.981299) (width 0.25) (layer "B.Cu") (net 9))
 (segment (start 115.2271 42.14876) (end 114.102099 43.273761) (width 0.25) (layer "B.Cu") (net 9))
 (segment (start 115.77066 56.77154) (end 115.77066 52.422736) (width 0.25) (layer "B.Cu") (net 9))
 (segment (start 114.102099 61.981299) (end 117.63248 65.51168) (width 0.25) (layer "B.Cu") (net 9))
 (segment (start 120.7516 26.6065) (end 123.89104 26.6065) (width 0.25) (layer "F.Cu") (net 10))
 (segment (start 123.89104 26.6065) (end 123.89612 26.60142) (width 0.25) (layer "F.Cu") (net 10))
 (segment (start 120.7516 26.6065) (end 118.06936 26.6065) (width 0.25) (layer "B.Cu") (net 10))
 (segment (start 120.7516 50.00498) (end 119.726599 51.029981) (width 0.25) (layer "B.Cu") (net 10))
 (segment (start 120.81002 49.94656) (end 120.7516 50.00498) (width 0.25) (layer "B.Cu") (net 10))
 (segment (start 118.06936 26.6065) (end 115.2271 29.44876) (width 0.25) (layer "B.Cu") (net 10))
 (segment (start 123.89612 49.94656) (end 122.871119 48.921559) (width 0.25) (layer "B.Cu") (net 10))
 (segment (start 122.794919 95.728679) (end 123.81992 96.75368) (width 0.25) (layer "B.Cu") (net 10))
 (segment (start 123.89612 73.3679) (end 122.794919 74.469101) (width 0.25) (layer "B.Cu") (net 10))
 (segment (start 120.7516 73.3679) (end 123.89612 73.3679) (width 0.25) (layer "B.Cu") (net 10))
 (segment (start 120.69572 96.75368) (end 120.6754 96.73336) (width 0.25) (layer "B.Cu") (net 10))
 (segment (start 123.81992 96.75368) (end 120.69572 96.75368) (width 0.25) (layer "B.Cu") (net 10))
 (segment (start 122.871119 27.626421) (end 123.89612 26.60142) (width 0.25) (layer "B.Cu") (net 10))
 (segment (start 119.726599 72.342899) (end 120.7516 73.3679) (width 0.25) (layer "B.Cu") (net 10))
 (segment (start 122.794919 74.469101) (end 122.794919 95.728679) (width 0.25) (layer "B.Cu") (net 10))
 (segment (start 123.89612 49.94656) (end 120.81002 49.94656) (width 0.25) (layer "B.Cu") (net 10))
 (segment (start 122.871119 48.921559) (end 122.871119 27.626421) (width 0.25) (layer "B.Cu") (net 10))
 (segment (start 119.726599 51.029981) (end 119.726599 72.342899) (width 0.25) (layer "B.Cu") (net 10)))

